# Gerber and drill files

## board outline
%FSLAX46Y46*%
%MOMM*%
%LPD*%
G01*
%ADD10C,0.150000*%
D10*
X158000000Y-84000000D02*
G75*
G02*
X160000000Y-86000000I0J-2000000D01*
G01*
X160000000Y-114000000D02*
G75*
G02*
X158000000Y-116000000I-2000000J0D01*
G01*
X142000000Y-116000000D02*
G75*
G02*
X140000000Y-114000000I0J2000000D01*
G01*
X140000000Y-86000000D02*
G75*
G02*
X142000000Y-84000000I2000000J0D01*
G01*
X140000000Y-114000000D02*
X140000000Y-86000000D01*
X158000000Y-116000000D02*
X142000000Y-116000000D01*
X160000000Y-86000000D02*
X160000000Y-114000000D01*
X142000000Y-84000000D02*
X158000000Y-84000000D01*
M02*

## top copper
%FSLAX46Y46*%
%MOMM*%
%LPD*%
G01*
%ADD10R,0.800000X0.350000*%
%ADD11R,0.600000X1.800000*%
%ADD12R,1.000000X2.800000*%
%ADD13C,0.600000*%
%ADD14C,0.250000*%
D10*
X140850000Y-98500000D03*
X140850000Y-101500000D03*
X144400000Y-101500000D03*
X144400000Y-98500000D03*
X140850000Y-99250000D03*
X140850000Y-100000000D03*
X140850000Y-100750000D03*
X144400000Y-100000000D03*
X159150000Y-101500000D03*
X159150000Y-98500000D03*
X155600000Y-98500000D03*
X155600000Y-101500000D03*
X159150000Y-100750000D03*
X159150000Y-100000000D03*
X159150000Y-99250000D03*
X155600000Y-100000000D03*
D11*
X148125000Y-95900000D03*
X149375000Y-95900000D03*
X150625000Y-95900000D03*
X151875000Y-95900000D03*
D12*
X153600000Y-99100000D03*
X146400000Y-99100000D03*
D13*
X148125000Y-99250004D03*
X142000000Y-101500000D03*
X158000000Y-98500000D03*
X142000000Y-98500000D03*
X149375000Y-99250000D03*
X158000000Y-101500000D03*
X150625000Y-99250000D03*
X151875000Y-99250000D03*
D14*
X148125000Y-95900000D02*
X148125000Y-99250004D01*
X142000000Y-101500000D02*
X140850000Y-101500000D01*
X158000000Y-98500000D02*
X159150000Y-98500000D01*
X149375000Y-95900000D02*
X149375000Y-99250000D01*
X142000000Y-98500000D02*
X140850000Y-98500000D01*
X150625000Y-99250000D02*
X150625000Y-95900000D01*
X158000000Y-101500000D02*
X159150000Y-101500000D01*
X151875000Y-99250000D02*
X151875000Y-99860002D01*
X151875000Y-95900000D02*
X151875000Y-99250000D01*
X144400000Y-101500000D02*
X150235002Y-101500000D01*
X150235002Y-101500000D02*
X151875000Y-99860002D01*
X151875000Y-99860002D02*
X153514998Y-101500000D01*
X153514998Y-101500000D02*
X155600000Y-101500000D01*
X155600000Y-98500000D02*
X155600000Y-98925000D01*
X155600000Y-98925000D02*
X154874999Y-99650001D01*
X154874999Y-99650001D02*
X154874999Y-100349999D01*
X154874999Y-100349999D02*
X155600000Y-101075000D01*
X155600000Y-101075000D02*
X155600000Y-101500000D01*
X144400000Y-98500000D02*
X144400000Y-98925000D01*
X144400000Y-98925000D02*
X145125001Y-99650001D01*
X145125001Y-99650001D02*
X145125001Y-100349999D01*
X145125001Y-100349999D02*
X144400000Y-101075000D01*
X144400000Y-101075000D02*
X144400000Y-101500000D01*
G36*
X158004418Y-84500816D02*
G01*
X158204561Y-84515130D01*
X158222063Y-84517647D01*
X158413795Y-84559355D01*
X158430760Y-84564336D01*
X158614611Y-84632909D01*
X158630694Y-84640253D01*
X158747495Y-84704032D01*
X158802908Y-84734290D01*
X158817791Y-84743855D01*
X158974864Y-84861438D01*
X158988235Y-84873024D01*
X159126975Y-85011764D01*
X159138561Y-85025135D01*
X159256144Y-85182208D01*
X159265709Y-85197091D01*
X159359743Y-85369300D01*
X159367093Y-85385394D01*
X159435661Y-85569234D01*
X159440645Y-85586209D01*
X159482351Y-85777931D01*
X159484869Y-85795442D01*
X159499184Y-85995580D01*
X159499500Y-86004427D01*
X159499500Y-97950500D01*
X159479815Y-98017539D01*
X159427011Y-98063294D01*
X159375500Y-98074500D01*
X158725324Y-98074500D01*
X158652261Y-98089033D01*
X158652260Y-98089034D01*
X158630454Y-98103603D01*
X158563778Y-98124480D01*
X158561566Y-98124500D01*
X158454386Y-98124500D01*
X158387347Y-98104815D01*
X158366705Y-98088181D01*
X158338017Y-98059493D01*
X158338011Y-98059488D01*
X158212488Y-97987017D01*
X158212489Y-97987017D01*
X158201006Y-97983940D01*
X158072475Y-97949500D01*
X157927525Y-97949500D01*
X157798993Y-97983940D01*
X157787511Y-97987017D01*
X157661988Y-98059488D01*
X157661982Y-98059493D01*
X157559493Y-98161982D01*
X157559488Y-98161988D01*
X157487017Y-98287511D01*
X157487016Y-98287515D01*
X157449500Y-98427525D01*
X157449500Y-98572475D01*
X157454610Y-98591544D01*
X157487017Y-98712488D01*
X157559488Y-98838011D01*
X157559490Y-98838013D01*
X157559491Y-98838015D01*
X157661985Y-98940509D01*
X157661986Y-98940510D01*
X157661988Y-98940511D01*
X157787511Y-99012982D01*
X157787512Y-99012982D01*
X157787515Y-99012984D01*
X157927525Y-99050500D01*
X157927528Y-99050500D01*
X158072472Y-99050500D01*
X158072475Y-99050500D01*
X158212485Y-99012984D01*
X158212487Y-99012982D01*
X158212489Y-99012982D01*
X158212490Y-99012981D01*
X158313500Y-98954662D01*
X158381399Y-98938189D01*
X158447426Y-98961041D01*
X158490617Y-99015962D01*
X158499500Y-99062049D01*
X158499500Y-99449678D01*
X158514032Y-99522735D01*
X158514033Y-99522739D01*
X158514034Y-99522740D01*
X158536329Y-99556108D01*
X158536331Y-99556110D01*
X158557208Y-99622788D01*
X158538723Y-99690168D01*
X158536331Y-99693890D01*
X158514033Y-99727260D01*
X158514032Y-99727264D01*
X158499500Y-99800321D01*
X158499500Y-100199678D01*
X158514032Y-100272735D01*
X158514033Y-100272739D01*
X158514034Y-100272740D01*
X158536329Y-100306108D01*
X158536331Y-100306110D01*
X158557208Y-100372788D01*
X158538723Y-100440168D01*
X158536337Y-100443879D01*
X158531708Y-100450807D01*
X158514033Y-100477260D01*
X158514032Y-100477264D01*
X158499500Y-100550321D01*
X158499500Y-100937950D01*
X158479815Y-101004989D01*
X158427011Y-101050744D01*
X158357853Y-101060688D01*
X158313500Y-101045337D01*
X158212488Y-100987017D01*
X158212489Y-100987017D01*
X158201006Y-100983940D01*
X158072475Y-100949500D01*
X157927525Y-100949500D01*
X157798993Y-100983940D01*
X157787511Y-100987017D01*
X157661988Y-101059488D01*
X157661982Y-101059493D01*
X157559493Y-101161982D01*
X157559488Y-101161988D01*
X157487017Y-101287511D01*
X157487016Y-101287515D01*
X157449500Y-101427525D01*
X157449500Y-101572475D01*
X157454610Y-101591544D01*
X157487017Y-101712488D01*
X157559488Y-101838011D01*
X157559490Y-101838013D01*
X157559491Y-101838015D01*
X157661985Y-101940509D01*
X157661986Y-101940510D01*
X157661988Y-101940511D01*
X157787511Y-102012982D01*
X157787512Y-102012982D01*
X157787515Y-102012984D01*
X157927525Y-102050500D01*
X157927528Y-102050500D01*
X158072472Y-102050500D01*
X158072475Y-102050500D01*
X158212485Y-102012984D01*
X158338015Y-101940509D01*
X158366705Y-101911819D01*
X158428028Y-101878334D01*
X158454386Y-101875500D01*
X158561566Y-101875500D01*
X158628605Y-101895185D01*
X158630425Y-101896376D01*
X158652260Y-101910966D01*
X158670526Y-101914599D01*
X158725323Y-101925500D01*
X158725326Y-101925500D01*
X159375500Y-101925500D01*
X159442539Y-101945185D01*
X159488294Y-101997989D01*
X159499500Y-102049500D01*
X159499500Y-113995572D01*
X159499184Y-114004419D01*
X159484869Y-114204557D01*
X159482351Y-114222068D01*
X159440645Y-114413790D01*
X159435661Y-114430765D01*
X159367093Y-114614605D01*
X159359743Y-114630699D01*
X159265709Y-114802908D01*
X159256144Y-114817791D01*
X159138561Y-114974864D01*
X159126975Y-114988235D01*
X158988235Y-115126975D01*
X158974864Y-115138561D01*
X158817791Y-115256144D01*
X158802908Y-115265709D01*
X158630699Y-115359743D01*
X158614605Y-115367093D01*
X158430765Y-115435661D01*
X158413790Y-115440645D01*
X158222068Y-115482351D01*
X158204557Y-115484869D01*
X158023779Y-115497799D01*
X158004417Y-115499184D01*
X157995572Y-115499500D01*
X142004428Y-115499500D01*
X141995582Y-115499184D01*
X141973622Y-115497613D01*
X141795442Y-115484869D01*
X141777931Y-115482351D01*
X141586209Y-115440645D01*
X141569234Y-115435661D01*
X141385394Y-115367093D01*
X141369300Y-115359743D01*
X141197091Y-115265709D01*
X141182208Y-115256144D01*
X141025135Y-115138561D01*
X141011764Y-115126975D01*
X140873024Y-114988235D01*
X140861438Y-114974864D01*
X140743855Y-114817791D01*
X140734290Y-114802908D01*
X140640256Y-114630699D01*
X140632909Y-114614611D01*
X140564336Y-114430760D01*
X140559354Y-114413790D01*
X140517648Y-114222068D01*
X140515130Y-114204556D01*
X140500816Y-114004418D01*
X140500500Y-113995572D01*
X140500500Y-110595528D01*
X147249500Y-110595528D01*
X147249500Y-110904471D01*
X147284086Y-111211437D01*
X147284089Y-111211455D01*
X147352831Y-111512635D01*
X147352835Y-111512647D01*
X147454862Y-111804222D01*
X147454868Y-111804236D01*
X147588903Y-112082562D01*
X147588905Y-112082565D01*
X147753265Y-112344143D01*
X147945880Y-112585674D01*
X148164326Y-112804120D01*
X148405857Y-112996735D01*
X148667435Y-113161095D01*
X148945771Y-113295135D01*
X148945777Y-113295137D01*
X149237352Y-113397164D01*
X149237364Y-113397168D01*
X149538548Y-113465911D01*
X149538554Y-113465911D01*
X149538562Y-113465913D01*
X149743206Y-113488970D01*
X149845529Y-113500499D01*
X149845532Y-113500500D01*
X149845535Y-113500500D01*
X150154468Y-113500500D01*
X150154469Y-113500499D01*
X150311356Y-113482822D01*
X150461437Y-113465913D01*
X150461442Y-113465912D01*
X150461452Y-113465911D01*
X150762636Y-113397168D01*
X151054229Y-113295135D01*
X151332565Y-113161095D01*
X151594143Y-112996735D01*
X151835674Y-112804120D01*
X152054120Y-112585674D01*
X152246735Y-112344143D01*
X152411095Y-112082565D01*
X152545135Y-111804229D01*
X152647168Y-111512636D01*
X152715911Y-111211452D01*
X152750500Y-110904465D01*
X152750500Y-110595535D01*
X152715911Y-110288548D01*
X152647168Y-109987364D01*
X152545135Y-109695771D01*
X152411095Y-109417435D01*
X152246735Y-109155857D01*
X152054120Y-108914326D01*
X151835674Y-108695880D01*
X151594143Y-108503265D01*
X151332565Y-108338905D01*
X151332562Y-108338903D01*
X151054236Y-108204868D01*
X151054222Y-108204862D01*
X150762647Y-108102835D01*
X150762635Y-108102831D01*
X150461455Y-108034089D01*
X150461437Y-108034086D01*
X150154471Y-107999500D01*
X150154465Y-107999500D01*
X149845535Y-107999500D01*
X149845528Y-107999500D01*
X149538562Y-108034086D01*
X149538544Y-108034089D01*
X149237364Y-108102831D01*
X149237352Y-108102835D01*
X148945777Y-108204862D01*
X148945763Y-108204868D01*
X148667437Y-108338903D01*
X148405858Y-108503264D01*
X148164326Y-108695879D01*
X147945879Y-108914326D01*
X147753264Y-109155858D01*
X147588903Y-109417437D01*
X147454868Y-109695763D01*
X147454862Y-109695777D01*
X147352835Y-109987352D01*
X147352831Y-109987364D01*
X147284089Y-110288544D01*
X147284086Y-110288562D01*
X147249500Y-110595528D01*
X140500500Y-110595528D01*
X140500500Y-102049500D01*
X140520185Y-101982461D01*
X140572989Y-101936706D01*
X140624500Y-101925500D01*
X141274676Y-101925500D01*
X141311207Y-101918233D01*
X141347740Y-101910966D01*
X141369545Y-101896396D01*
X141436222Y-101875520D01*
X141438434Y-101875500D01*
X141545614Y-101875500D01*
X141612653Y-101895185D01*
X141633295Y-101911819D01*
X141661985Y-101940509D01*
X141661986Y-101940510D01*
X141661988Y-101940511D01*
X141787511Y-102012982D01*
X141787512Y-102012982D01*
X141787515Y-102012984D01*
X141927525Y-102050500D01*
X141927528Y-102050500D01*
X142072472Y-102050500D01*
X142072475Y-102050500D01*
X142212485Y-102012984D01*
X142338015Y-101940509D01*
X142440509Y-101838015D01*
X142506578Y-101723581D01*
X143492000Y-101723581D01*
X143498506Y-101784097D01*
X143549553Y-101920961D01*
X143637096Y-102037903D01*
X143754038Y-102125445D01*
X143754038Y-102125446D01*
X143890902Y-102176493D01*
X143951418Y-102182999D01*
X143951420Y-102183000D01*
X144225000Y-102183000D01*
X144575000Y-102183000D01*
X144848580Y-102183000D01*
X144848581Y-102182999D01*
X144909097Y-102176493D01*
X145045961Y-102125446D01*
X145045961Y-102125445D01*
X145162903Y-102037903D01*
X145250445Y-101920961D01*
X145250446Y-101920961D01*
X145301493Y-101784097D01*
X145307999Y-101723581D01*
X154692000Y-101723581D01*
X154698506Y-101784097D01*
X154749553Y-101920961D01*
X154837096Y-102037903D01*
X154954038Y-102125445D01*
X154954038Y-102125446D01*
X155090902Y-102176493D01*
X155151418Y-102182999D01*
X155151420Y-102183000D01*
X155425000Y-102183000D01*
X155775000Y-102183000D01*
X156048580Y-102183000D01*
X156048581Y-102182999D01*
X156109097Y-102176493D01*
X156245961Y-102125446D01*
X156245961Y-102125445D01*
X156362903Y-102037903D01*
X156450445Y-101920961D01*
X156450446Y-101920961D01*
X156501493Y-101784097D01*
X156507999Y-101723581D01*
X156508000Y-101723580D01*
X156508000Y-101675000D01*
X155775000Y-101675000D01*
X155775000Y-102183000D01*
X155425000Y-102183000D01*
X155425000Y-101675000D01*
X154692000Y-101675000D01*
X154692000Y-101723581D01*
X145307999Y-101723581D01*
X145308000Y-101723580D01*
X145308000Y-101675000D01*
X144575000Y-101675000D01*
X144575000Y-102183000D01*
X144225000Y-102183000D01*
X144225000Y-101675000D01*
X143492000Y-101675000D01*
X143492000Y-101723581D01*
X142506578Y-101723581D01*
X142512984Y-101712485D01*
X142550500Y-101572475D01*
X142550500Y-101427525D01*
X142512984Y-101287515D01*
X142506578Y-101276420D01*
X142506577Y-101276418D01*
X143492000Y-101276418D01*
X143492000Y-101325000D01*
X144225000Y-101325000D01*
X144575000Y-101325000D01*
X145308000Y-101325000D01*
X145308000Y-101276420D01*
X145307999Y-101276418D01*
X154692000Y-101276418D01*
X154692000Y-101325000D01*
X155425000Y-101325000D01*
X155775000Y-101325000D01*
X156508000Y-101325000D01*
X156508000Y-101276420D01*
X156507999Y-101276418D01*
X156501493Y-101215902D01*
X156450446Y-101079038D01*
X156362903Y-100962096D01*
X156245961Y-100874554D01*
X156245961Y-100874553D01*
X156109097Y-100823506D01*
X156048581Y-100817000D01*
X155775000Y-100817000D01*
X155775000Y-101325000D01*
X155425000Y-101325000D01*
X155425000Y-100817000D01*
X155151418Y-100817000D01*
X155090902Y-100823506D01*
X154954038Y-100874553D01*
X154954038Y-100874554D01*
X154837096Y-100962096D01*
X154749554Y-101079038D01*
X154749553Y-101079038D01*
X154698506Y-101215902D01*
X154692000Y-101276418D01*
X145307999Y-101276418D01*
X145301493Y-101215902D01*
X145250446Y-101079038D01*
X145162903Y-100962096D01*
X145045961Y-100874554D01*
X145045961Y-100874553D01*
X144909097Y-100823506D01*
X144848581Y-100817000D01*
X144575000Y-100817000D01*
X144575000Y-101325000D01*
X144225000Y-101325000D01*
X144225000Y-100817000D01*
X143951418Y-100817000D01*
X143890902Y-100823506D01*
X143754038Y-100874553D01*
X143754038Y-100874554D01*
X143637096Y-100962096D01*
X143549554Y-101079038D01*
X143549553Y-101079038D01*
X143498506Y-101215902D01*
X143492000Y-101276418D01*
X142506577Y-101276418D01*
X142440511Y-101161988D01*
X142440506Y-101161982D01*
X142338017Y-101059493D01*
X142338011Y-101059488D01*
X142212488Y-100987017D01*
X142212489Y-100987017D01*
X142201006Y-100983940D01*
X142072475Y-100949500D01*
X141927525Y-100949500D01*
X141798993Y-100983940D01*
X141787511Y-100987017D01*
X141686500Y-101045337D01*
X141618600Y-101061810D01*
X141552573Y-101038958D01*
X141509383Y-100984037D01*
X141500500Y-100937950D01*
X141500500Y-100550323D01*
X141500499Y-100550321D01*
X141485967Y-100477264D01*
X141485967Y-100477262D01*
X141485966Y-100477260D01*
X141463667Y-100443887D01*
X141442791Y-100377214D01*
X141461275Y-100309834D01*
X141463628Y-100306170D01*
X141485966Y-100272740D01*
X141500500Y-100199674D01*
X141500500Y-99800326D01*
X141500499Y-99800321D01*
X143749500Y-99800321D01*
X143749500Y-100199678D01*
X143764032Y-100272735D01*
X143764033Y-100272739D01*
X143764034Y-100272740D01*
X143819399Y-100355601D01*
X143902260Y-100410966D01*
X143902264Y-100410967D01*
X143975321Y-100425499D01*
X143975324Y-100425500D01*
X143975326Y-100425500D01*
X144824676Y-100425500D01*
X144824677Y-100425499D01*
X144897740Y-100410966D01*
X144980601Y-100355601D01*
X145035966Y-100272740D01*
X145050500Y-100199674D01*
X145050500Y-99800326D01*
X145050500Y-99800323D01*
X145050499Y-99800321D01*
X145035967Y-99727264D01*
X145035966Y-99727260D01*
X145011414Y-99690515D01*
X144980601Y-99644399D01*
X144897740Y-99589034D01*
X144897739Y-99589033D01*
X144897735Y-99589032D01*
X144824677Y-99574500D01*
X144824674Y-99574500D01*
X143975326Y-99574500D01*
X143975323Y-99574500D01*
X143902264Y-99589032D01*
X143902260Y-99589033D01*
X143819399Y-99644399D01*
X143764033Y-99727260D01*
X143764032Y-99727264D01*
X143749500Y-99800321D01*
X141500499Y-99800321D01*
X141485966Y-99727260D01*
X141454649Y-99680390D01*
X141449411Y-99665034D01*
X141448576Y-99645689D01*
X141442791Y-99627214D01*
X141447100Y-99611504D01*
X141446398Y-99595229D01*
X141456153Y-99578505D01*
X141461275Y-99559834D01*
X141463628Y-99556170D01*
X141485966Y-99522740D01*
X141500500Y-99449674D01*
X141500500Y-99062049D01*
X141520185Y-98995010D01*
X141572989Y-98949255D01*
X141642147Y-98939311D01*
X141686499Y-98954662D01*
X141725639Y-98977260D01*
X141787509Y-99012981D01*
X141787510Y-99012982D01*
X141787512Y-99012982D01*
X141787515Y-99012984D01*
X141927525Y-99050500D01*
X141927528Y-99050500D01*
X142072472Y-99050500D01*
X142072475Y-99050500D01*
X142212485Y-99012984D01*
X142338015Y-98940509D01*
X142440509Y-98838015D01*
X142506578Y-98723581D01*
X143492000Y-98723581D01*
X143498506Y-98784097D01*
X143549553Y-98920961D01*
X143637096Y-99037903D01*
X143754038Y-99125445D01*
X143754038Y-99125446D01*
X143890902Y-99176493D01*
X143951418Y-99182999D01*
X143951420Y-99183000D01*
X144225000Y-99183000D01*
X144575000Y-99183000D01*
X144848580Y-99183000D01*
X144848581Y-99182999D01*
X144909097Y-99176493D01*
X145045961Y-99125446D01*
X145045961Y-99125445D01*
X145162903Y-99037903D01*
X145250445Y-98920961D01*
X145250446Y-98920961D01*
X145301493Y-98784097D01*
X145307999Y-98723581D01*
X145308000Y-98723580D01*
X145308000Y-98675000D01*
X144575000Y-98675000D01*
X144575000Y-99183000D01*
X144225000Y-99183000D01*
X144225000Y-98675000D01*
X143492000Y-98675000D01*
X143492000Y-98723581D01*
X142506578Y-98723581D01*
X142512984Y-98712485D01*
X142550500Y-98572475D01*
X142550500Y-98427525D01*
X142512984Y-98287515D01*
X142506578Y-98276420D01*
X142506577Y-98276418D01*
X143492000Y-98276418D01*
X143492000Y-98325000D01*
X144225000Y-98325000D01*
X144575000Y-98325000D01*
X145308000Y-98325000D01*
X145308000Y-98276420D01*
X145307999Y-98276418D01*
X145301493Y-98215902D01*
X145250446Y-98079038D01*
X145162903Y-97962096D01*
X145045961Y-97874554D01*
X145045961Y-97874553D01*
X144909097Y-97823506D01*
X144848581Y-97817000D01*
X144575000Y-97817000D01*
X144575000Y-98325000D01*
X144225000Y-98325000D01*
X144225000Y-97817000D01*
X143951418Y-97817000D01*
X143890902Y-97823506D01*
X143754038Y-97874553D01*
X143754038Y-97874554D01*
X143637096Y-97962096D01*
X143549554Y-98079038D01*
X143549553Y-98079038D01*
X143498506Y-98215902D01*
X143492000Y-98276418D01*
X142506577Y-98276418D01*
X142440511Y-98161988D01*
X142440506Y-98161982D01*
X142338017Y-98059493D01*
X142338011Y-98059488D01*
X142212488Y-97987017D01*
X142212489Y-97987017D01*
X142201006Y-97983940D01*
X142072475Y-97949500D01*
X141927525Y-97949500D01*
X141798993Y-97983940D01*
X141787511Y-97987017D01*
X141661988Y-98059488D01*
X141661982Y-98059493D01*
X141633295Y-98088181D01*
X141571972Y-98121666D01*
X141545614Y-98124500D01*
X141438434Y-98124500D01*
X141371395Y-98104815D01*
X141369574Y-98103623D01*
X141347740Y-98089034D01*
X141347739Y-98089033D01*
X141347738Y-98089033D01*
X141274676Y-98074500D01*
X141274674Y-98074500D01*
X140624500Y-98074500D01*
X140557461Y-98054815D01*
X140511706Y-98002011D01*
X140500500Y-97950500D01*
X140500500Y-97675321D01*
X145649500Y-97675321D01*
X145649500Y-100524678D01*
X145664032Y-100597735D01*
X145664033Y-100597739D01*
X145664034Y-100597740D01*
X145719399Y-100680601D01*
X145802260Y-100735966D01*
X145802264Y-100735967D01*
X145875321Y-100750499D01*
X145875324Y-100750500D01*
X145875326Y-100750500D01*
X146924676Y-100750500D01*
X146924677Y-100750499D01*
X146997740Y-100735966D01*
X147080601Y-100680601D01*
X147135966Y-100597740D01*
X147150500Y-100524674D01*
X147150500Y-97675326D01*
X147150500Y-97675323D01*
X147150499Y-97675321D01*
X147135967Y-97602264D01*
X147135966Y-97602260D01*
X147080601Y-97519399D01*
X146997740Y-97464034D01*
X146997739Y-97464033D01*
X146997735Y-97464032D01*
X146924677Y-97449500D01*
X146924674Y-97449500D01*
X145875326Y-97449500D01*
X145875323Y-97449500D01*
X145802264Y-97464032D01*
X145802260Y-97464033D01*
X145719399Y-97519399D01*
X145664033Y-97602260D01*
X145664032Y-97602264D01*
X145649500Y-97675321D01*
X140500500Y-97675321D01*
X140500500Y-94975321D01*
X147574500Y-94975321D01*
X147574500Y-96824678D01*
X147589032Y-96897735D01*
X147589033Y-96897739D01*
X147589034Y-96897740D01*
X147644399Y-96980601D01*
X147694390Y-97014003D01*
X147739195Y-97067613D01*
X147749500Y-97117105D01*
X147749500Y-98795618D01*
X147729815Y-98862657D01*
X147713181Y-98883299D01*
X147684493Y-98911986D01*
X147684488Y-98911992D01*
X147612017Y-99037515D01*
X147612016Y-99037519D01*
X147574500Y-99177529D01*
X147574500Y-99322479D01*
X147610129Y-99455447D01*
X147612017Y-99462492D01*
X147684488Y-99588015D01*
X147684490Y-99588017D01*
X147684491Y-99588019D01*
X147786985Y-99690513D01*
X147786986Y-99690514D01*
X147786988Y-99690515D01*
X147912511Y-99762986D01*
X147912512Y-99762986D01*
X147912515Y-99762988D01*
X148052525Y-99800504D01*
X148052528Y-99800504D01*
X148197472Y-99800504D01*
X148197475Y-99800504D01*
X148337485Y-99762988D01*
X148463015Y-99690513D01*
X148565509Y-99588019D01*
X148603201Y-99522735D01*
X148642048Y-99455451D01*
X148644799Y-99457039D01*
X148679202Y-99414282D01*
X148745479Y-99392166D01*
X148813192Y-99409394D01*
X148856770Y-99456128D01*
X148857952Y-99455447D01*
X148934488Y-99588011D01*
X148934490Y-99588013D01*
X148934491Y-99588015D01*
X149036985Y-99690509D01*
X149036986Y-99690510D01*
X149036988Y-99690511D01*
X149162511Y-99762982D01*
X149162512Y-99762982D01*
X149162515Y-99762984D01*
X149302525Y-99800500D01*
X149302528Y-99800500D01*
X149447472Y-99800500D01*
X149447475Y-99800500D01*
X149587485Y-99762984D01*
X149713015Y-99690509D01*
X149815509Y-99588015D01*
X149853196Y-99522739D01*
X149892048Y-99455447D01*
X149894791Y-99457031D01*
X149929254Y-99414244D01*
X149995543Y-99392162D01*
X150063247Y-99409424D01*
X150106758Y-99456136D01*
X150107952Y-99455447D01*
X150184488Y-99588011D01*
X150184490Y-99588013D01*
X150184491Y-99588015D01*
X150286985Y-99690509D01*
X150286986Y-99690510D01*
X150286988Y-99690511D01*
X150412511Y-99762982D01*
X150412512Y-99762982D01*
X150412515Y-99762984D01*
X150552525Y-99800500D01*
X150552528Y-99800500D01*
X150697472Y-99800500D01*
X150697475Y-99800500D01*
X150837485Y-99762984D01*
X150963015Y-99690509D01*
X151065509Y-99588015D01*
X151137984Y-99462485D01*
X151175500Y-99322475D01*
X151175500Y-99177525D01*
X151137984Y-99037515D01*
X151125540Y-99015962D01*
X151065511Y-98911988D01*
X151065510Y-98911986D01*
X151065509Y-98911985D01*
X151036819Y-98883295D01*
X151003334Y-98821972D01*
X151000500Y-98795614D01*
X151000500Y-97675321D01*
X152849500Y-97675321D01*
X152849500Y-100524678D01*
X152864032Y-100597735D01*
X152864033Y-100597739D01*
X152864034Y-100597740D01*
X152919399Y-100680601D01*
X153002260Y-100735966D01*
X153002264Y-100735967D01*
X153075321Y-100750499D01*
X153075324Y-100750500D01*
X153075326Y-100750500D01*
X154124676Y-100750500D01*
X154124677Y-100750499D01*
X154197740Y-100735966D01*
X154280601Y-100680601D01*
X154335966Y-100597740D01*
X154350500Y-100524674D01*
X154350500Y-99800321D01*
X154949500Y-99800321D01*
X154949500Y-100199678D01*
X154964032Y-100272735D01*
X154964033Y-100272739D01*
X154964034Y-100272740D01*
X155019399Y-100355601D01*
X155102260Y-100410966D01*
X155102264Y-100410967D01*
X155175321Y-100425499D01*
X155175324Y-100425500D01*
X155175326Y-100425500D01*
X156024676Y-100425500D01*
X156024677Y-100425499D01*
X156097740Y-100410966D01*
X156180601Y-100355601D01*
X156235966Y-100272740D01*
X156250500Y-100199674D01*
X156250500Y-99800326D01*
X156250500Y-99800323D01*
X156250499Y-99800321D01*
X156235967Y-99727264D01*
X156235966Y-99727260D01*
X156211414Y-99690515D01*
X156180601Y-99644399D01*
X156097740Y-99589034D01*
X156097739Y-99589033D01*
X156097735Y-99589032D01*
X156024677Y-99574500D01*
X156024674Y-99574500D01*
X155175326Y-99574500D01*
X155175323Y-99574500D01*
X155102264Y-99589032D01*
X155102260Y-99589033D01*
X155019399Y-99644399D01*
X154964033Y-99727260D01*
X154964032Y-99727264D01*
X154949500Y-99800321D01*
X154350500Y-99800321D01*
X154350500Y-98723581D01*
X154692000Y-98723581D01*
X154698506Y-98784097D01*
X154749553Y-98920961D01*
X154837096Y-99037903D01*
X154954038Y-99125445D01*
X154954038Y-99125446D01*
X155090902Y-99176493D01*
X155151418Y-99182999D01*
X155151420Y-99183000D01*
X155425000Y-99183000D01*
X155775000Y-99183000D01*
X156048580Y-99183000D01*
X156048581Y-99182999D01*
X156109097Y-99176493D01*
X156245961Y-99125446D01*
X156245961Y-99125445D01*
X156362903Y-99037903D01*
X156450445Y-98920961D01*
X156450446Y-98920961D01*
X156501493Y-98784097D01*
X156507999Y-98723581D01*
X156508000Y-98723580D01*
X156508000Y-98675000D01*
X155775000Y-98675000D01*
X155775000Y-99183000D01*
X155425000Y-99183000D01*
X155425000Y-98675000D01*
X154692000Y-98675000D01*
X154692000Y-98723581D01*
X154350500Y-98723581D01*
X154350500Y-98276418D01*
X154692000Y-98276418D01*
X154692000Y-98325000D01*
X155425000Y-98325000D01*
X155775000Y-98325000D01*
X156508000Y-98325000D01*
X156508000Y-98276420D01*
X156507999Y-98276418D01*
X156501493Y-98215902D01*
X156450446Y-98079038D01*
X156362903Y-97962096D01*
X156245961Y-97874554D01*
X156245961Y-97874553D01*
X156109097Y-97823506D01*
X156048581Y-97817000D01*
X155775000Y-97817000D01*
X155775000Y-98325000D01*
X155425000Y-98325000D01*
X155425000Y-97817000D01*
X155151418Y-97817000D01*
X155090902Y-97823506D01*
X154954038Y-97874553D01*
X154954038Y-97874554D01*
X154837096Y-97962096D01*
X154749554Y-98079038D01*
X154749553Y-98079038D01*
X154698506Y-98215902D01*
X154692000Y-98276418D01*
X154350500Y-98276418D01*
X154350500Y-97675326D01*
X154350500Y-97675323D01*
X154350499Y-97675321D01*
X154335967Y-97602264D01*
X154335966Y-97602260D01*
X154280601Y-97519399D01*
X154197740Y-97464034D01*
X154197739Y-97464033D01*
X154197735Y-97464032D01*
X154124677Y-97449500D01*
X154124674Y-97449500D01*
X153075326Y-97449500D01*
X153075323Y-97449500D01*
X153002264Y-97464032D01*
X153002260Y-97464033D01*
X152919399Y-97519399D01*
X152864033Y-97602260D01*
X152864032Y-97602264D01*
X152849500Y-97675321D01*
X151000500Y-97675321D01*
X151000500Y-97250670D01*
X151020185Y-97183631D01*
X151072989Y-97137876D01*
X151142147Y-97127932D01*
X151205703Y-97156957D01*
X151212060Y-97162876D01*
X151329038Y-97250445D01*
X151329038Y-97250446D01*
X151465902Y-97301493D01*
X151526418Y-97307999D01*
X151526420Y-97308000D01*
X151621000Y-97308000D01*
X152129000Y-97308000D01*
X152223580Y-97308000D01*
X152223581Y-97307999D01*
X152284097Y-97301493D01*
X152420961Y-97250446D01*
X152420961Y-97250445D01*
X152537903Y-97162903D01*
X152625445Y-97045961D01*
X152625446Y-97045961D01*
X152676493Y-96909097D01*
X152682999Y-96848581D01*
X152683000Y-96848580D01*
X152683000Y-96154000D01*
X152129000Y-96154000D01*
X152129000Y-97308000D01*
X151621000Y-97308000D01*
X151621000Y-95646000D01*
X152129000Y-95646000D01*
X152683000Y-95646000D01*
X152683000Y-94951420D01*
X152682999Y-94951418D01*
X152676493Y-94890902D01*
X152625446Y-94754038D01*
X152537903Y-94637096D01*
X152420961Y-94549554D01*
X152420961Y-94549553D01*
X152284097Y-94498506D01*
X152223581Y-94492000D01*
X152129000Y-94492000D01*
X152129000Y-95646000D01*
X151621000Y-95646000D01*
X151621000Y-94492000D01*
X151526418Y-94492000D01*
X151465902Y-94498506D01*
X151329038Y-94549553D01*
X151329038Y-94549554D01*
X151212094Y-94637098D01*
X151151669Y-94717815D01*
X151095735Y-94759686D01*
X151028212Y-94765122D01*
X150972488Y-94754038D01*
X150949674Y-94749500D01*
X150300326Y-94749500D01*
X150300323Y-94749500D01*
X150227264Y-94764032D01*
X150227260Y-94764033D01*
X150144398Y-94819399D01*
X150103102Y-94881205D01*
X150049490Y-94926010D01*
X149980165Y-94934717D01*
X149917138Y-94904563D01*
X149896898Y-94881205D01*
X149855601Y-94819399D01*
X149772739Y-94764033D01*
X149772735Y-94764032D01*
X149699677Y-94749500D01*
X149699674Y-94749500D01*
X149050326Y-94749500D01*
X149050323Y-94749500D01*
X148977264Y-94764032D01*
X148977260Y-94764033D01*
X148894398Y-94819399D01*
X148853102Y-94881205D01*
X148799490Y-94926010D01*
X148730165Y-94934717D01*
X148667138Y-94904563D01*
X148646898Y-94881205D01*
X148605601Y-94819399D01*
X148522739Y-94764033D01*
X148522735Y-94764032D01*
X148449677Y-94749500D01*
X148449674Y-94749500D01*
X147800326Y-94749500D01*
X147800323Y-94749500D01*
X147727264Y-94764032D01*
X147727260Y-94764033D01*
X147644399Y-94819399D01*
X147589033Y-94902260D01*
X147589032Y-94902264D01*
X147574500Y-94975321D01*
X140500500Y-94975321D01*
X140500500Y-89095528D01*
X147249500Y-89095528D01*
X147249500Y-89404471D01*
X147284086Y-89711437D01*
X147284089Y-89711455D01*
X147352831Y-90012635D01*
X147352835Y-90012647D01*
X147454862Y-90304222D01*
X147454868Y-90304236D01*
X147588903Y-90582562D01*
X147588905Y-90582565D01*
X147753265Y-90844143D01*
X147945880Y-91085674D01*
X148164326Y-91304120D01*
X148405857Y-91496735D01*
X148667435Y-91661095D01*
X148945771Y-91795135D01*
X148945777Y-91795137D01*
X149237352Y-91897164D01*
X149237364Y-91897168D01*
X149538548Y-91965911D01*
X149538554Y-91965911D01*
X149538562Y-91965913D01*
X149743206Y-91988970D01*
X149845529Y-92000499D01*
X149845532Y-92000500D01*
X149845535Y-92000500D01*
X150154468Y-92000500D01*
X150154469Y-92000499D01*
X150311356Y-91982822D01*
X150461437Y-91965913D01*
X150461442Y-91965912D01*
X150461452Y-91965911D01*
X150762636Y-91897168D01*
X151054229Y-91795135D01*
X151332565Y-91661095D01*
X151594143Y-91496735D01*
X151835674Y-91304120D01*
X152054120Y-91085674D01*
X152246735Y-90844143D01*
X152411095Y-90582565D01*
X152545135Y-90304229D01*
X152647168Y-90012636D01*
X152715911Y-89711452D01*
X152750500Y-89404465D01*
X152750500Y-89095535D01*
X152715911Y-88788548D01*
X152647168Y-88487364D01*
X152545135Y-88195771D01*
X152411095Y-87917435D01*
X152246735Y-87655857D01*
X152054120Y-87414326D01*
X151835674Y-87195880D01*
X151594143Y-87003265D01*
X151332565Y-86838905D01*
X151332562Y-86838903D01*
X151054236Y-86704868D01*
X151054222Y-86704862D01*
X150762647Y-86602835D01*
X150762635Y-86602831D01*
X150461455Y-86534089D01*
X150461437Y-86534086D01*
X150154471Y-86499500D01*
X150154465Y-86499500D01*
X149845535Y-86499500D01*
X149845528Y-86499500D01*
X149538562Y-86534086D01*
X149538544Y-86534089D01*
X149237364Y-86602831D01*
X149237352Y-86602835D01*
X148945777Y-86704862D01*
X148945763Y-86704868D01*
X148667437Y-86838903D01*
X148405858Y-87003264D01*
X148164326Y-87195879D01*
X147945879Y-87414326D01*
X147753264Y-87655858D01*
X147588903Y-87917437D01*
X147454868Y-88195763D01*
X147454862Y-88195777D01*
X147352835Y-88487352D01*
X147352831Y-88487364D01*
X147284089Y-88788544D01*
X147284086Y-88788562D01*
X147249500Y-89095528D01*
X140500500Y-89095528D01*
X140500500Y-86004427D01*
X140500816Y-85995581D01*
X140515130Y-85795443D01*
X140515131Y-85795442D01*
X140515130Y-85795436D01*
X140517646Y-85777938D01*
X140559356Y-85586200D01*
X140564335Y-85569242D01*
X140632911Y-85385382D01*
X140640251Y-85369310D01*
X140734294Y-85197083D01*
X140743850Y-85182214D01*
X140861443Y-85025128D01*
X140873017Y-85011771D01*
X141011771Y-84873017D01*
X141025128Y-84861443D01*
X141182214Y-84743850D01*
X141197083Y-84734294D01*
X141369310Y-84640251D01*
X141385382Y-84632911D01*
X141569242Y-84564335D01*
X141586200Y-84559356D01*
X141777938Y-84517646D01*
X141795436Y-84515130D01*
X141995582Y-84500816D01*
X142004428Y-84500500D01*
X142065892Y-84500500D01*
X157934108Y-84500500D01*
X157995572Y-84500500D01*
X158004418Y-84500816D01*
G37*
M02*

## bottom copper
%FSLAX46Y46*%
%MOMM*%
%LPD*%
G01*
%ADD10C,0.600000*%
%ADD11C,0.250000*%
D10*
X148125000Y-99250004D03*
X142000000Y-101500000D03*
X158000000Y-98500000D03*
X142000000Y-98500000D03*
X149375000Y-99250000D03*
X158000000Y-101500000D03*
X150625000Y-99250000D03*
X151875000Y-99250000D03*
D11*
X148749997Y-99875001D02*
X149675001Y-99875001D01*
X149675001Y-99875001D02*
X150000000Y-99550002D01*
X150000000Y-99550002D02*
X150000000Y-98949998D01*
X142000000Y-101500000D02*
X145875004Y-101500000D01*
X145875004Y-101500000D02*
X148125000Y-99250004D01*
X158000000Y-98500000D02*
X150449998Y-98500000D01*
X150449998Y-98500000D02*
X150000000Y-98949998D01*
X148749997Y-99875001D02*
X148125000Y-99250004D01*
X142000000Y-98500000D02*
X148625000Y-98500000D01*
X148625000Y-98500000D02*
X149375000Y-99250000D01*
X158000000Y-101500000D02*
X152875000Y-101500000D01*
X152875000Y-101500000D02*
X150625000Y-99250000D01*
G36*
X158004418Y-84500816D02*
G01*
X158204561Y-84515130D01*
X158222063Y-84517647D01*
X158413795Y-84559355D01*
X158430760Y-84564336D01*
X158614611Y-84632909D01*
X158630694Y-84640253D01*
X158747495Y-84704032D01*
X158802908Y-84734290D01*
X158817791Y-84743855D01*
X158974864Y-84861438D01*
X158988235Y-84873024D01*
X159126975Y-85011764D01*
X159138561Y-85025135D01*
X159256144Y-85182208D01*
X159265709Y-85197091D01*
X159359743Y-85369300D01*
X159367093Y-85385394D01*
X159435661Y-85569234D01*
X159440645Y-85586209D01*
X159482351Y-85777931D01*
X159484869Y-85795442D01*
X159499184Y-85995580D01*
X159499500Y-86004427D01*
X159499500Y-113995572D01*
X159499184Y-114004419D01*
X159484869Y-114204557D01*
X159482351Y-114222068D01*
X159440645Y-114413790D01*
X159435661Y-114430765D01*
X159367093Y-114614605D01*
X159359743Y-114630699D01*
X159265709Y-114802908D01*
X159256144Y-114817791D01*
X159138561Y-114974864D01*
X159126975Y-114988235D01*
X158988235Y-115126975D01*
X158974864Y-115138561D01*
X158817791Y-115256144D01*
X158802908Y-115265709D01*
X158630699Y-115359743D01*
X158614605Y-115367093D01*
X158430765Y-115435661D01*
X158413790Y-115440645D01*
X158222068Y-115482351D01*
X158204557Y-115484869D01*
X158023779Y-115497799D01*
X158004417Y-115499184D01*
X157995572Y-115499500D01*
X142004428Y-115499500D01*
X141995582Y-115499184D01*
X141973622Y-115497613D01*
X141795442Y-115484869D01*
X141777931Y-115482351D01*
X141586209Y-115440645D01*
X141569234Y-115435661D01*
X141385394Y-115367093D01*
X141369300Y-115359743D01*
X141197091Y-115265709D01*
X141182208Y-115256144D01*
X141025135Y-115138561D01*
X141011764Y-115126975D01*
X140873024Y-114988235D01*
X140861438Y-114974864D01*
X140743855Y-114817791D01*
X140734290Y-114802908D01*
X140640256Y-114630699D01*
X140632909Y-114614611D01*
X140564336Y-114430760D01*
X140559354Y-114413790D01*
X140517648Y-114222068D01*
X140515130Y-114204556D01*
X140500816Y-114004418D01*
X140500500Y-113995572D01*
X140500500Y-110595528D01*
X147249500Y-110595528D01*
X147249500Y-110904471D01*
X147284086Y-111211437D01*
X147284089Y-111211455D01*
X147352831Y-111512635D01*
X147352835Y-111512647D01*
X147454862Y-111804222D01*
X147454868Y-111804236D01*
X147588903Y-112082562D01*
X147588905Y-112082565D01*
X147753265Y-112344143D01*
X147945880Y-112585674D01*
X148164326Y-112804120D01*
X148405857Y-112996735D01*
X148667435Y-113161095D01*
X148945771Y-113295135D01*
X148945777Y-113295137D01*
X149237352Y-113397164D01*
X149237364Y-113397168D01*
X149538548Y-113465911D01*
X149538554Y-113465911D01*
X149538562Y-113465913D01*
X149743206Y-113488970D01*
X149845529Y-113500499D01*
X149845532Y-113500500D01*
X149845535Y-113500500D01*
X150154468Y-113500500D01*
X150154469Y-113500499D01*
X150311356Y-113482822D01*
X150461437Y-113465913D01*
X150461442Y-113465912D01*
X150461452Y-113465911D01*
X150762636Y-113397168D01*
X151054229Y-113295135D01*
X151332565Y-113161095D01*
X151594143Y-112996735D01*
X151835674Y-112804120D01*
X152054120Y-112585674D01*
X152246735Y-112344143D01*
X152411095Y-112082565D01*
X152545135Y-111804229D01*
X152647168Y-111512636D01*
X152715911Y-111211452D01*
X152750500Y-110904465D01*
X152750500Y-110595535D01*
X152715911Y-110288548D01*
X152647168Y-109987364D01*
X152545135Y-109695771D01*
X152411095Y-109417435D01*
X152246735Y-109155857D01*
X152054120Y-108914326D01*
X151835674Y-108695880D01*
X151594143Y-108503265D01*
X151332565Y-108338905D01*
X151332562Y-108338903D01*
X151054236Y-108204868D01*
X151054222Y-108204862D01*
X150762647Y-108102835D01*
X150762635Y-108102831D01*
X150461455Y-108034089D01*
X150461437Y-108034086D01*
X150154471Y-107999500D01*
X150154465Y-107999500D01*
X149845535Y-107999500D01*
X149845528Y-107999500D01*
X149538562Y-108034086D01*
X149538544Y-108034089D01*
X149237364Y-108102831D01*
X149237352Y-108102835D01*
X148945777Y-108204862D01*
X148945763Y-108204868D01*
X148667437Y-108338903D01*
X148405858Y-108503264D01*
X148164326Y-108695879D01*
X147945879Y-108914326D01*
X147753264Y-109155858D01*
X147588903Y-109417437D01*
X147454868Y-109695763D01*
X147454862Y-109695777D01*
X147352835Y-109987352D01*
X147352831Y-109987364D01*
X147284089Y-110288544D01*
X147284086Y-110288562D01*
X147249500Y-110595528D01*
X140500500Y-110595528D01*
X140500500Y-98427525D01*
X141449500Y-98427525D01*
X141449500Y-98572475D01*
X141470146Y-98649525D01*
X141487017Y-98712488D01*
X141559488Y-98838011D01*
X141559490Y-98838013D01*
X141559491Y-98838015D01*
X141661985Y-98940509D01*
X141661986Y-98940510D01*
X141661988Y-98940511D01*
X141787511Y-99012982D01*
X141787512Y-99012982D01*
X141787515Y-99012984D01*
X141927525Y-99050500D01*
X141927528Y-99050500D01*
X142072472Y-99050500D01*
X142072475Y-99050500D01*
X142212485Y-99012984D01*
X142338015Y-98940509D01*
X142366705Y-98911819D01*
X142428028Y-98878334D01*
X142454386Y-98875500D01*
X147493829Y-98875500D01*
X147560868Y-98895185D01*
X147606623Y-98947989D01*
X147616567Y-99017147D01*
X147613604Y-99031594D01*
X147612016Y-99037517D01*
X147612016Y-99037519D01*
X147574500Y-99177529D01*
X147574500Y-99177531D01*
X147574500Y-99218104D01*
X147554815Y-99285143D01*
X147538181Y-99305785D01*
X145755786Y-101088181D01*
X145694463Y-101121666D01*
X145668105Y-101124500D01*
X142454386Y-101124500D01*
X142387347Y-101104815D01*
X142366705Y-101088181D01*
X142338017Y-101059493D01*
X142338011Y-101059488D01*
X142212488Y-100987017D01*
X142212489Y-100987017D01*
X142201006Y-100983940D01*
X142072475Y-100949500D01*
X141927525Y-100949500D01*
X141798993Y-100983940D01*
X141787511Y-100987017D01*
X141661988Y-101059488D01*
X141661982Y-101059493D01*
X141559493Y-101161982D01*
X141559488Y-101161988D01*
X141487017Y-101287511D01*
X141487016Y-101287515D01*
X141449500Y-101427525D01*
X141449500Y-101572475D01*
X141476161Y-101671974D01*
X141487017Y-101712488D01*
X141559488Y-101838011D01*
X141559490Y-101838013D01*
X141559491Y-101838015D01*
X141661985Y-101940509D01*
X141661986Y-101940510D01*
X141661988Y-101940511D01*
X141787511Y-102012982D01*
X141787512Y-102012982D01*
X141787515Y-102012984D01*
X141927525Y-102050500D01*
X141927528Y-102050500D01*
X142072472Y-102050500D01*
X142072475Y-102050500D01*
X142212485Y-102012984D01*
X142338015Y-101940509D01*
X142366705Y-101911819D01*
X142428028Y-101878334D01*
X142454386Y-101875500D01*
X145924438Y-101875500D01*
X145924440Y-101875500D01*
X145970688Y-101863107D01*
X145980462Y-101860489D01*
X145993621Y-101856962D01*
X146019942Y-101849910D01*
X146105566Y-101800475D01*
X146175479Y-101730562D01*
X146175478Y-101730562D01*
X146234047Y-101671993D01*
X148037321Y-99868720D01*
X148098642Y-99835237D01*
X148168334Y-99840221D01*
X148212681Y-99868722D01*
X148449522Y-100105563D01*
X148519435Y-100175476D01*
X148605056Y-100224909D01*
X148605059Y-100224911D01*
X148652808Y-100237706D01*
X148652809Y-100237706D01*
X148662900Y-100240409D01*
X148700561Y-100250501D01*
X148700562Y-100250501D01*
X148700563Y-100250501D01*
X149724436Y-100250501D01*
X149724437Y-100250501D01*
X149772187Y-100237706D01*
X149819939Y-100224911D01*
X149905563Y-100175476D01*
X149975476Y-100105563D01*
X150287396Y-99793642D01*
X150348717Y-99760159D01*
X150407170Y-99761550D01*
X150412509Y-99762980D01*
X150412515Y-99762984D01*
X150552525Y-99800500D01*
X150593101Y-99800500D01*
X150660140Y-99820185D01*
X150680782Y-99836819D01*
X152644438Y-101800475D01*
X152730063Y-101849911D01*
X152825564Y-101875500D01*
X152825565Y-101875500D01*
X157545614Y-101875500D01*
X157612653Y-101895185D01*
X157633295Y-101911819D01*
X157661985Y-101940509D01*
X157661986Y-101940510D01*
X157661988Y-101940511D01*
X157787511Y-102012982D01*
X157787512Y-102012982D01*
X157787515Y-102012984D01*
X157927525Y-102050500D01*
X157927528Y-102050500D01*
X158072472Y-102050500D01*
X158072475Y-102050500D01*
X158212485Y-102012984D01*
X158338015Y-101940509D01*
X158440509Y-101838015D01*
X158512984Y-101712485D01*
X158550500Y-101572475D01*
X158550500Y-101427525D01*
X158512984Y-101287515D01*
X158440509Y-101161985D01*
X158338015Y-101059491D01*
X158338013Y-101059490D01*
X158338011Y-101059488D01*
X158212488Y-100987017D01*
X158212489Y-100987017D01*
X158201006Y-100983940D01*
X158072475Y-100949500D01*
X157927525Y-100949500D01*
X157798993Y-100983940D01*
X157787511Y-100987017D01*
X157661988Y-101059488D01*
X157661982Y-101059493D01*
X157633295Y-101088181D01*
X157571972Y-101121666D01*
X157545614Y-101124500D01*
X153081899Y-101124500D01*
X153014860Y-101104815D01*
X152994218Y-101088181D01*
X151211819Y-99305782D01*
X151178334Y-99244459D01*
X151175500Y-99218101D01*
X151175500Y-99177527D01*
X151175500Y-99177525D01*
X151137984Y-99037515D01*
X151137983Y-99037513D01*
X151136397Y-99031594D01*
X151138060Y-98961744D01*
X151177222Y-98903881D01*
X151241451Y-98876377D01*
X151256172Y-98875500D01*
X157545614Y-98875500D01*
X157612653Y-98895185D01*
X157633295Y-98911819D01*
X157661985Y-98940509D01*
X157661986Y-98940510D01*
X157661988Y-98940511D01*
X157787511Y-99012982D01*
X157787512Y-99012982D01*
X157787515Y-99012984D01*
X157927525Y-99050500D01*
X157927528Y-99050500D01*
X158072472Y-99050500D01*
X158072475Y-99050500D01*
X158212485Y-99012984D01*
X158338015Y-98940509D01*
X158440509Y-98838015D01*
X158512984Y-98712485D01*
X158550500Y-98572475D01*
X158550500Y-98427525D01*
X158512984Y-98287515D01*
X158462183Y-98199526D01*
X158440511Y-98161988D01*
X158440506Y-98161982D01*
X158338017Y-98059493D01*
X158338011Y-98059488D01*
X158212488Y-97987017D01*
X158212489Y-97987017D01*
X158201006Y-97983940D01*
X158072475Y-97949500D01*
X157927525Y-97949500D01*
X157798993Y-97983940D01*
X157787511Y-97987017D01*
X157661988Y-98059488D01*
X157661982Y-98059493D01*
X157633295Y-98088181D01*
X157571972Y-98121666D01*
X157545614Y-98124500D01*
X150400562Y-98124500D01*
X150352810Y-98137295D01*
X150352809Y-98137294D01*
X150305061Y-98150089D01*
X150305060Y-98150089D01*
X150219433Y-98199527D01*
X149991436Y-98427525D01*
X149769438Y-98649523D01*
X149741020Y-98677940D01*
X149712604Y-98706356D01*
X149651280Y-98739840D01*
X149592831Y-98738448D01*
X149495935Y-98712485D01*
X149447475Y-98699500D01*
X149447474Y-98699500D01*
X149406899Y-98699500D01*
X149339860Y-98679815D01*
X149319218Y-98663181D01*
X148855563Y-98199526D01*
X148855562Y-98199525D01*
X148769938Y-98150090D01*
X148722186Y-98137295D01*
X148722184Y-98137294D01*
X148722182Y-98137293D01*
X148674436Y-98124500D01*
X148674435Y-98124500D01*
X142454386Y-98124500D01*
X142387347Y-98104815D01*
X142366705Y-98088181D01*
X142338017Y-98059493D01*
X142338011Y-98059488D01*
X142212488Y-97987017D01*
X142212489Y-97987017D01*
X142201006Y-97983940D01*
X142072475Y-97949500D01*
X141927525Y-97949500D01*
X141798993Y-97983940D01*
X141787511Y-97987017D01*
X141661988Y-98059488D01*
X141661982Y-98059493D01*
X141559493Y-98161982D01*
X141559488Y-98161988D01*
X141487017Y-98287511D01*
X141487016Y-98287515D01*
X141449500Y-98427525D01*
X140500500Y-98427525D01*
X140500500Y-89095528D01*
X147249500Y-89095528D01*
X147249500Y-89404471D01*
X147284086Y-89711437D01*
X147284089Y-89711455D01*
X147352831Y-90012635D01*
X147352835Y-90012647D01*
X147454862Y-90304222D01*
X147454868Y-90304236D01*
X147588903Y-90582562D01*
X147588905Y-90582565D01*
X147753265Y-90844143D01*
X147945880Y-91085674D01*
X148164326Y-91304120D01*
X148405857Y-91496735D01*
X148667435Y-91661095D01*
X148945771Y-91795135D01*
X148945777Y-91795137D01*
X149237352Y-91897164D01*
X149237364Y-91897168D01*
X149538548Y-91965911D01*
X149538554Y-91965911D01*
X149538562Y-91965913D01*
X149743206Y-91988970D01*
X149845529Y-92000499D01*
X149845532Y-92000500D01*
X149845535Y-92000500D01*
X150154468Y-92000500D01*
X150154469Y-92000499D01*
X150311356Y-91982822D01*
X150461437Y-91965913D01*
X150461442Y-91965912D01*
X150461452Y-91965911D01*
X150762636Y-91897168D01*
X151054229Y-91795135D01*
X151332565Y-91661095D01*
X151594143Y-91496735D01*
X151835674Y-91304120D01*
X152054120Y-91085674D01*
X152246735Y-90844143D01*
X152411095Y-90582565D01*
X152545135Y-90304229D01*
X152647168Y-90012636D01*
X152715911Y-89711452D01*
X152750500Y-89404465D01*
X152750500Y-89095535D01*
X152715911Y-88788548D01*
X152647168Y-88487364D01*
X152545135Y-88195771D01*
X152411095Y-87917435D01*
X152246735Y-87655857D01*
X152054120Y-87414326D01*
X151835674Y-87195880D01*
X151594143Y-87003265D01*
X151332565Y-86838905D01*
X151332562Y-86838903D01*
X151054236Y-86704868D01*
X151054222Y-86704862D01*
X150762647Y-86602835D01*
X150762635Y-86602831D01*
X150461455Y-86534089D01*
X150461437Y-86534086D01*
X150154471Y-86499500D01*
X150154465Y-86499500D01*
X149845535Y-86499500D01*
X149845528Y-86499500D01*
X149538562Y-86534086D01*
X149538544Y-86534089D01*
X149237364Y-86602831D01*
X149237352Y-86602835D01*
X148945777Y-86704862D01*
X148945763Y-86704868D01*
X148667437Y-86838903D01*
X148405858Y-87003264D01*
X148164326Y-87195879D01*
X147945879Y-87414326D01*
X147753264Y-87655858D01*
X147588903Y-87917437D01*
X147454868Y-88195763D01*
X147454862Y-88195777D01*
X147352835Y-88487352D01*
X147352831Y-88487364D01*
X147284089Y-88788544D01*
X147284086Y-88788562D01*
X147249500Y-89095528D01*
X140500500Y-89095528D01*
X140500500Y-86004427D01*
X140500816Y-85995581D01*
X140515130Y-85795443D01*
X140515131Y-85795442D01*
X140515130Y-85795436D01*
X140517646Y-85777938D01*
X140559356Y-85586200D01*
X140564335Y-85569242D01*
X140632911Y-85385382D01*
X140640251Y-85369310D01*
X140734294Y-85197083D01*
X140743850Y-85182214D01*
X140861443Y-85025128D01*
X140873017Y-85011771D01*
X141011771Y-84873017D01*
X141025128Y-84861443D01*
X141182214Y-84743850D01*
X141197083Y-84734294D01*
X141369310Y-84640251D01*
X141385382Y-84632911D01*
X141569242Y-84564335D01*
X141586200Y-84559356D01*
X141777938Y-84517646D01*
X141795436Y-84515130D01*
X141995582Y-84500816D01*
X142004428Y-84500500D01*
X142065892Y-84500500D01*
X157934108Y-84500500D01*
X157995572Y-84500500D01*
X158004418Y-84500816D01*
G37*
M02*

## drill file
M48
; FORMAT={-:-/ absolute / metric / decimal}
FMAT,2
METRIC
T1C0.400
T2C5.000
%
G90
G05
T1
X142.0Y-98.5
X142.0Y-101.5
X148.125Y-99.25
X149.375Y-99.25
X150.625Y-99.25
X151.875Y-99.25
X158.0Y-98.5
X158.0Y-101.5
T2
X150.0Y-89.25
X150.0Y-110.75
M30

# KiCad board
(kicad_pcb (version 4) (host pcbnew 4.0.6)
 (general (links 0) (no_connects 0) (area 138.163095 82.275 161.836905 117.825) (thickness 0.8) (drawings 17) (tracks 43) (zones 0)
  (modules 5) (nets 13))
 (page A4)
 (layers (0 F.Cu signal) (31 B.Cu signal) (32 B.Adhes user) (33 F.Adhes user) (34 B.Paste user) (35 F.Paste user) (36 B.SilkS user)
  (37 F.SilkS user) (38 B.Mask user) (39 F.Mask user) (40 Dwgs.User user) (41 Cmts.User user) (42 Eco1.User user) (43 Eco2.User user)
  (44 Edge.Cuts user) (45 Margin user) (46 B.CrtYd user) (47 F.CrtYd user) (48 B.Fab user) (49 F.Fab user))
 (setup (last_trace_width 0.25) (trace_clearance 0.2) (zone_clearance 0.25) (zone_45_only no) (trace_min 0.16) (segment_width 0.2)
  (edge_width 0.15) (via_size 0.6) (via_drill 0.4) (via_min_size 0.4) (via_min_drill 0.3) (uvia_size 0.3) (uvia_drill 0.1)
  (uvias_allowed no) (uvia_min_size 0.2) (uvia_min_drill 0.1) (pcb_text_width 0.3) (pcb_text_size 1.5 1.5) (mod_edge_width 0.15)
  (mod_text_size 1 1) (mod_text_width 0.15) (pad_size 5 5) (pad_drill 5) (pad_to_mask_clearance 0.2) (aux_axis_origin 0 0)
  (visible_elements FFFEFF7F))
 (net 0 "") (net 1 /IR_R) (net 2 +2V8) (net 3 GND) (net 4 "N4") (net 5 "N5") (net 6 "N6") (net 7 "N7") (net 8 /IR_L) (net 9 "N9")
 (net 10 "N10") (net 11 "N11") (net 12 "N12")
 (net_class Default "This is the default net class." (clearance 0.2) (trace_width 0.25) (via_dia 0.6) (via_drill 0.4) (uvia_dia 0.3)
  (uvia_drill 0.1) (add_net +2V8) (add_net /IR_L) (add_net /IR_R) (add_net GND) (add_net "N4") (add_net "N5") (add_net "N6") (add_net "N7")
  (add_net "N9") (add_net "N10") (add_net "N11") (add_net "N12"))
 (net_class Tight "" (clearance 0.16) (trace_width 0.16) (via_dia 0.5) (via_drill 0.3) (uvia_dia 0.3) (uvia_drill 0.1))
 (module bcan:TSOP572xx (layer F.Cu) (at 142.625 100)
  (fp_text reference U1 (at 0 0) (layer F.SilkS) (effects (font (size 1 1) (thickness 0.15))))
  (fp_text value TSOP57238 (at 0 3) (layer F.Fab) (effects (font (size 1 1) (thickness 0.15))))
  (pad 1 smd rect (at -1.775 -1.5) (size 0.8 0.35) (layers F.Cu F.Paste F.Mask) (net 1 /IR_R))
  (pad 5 smd rect (at -1.775 1.5) (size 0.8 0.35) (layers F.Cu F.Paste F.Mask) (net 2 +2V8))
  (pad 6 smd rect (at 1.775 1.5) (size 0.8 0.35) (layers F.Cu F.Paste F.Mask) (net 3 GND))
  (pad 8 smd rect (at 1.775 -1.5) (size 0.8 0.35) (layers F.Cu F.Paste F.Mask) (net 3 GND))
  (pad 2 smd rect (at -1.775 -0.75) (size 0.8 0.35) (layers F.Cu F.Mask) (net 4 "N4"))
  (pad 3 smd rect (at -1.775 0) (size 0.8 0.35) (layers F.Cu F.Mask) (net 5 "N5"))
  (pad 4 smd rect (at -1.775 0.75) (size 0.8 0.35) (layers F.Cu F.Mask) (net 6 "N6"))
  (pad 7 smd rect (at 1.775 0) (size 0.8 0.35) (layers F.Cu F.Mask) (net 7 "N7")))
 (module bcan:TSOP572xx (layer F.Cu) (at 157.375 100 180)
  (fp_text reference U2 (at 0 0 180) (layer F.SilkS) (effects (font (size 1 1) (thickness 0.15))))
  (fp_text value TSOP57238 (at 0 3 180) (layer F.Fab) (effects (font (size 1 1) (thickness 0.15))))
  (pad 1 smd rect (at -1.775 -1.5 180) (size 0.8 0.35) (layers F.Cu F.Paste F.Mask) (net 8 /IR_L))
  (pad 5 smd rect (at -1.775 1.5 180) (size 0.8 0.35) (layers F.Cu F.Paste F.Mask) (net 2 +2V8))
  (pad 6 smd rect (at 1.775 1.5 180) (size 0.8 0.35) (layers F.Cu F.Paste F.Mask) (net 3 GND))
  (pad 8 smd rect (at 1.775 -1.5 180) (size 0.8 0.35) (layers F.Cu F.Paste F.Mask) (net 3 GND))
  (pad 2 smd rect (at -1.775 -0.75 180) (size 0.8 0.35) (layers F.Cu F.Mask) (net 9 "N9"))
  (pad 3 smd rect (at -1.775 0 180) (size 0.8 0.35) (layers F.Cu F.Mask) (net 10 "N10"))
  (pad 4 smd rect (at -1.775 0.75 180) (size 0.8 0.35) (layers F.Cu F.Mask) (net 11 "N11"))
  (pad 7 smd rect (at 1.775 0 180) (size 0.8 0.35) (layers F.Cu F.Mask) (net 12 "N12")))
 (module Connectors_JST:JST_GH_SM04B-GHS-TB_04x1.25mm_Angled (layer F.Cu) (at 150 97.5)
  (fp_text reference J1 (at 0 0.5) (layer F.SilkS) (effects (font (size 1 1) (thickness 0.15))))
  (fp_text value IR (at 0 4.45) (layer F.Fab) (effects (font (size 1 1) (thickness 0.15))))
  (pad 1 smd rect (at -1.875 -1.6) (size 0.6 1.8) (layers F.Cu F.Paste F.Mask) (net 2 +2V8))
  (pad 2 smd rect (at -0.625 -1.6) (size 0.6 1.8) (layers F.Cu F.Paste F.Mask) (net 1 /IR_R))
  (pad 3 smd rect (at 0.625 -1.6) (size 0.6 1.8) (layers F.Cu F.Paste F.Mask) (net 8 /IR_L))
  (pad 4 smd rect (at 1.875 -1.6) (size 0.6 1.8) (layers F.Cu F.Paste F.Mask) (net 3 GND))
  (pad "" smd rect (at 3.6 1.6) (size 1 2.8) (layers F.Cu F.Paste F.Mask))
  (pad "" smd rect (at -3.6 1.6) (size 1 2.8) (layers F.Cu F.Paste F.Mask)))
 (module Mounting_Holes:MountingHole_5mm (layer F.Cu) (at 150 89.25)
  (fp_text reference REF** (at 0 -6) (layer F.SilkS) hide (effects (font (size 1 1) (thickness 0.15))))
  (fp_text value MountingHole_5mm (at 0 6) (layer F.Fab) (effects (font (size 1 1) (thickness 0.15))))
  (pad 1 np_thru_hole circle (at 0 0) (size 5 5) (drill 5) (layers *.Cu *.Mask)))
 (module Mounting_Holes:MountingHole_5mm (layer F.Cu) (at 150 110.75)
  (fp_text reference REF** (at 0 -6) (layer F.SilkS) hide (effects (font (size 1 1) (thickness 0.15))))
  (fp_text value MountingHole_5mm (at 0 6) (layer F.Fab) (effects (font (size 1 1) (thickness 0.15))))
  (pad 1 np_thru_hole circle (at 0 0) (size 5 5) (drill 5) (layers *.Cu *.Mask)))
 (gr_arc (start 158 86) (end 158 84) (angle 90) (layer Edge.Cuts) (width 0.15))
 (gr_arc (start 158 114) (end 160 114) (angle 90) (layer Edge.Cuts) (width 0.15))
 (gr_arc (start 142 114) (end 142 116) (angle 90) (layer Edge.Cuts) (width 0.15))
 (gr_arc (start 142 86) (end 140 86) (angle 90) (layer Edge.Cuts) (width 0.15))
 (gr_line (start 140 114) (end 140 86) (layer Edge.Cuts) (width 0.15))
 (gr_line (start 158 116) (end 142 116) (layer Edge.Cuts) (width 0.15))
 (gr_line (start 160 86) (end 160 114) (layer Edge.Cuts) (width 0.15))
 (gr_line (start 142 84) (end 158 84) (layer Edge.Cuts) (width 0.15))
 (segment (start 148.749997 99.875001) (end 149.675001 99.875001) (width 0.25) (layer B.Cu) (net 2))
 (segment (start 149.675001 99.875001) (end 150 99.550002) (width 0.25) (layer B.Cu) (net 2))
 (segment (start 150 99.550002) (end 150 98.949998) (width 0.25) (layer B.Cu) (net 2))
 (segment (start 142 101.5) (end 145.875004 101.5) (width 0.25) (layer B.Cu) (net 2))
 (segment (start 145.875004 101.5) (end 148.125 99.250004) (width 0.25) (layer B.Cu) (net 2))
 (segment (start 158 98.5) (end 150.449998 98.5) (width 0.25) (layer B.Cu) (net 2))
 (segment (start 150.449998 98.5) (end 150 98.949998) (width 0.25) (layer B.Cu) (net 2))
 (segment (start 148.749997 99.875001) (end 148.125 99.250004) (width 0.25) (layer B.Cu) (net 2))
 (segment (start 148.125 95.9) (end 148.125 99.250004) (width 0.25) (layer F.Cu) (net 2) (status 10))
 (via (at 148.125 99.250004) (size 0.6) (drill 0.4) (layers F.Cu B.Cu) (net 2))
 (segment (start 142 101.5) (end 140.85 101.5) (width 0.25) (layer F.Cu) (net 2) (status 20))
 (via (at 142 101.5) (size 0.6) (drill 0.4) (layers F.Cu B.Cu) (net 2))
 (segment (start 158 98.5) (end 159.15 98.5) (width 0.25) (layer F.Cu) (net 2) (status 20))
 (via (at 158 98.5) (size 0.6) (drill 0.4) (layers F.Cu B.Cu) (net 2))
 (segment (start 142 98.5) (end 148.625 98.5) (width 0.25) (layer B.Cu) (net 1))
 (segment (start 148.625 98.5) (end 149.375 99.25) (width 0.25) (layer B.Cu) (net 1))
 (segment (start 149.375 95.9) (end 149.375 99.25) (width 0.25) (layer F.Cu) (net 1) (status 10))
 (segment (start 142 98.5) (end 140.85 98.5) (width 0.25) (layer F.Cu) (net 1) (status 20))
 (via (at 142 98.5) (size 0.6) (drill 0.4) (layers F.Cu B.Cu) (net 1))
 (via (at 149.375 99.25) (size 0.6) (drill 0.4) (layers F.Cu B.Cu) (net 1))
 (segment (start 150.625 99.25) (end 150.625 95.9) (width 0.25) (layer F.Cu) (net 8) (status 20))
 (segment (start 158 101.5) (end 152.875 101.5) (width 0.25) (layer B.Cu) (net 8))
 (segment (start 152.875 101.5) (end 150.625 99.25) (width 0.25) (layer B.Cu) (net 8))
 (segment (start 158 101.5) (end 159.15 101.5) (width 0.25) (layer F.Cu) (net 8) (status 20))
 (via (at 158 101.5) (size 0.6) (drill 0.4) (layers F.Cu B.Cu) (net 8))
 (via (at 150.625 99.25) (size 0.6) (drill 0.4) (layers F.Cu B.Cu) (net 8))
 (segment (start 151.875 99.25) (end 151.875 99.860002) (width 0.25) (layer F.Cu) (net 3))
 (segment (start 151.875 95.9) (end 151.875 99.25) (width 0.25) (layer F.Cu) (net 3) (status 10))
 (via (at 151.875 99.25) (size 0.6) (drill 0.4) (layers F.Cu B.Cu) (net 3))
 (segment (start 144.4 101.5) (end 150.235002 101.5) (width 0.25) (layer F.Cu) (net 3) (status 10))
 (segment (start 150.235002 101.5) (end 151.875 99.860002) (width 0.25) (layer F.Cu) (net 3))
 (segment (start 151.875 99.860002) (end 153.514998 101.5) (width 0.25) (layer F.Cu) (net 3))
 (segment (start 153.514998 101.5) (end 155.6 101.5) (width 0.25) (layer F.Cu) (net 3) (status 20))
 (segment (start 155.6 98.5) (end 155.6 98.925) (width 0.25) (layer F.Cu) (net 3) (status 10))
 (segment (start 155.6 98.925) (end 154.874999 99.650001) (width 0.25) (layer F.Cu) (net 3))
 (segment (start 154.874999 99.650001) (end 154.874999 100.349999) (width 0.25) (layer F.Cu) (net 3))
 (segment (start 154.874999 100.349999) (end 155.6 101.075) (width 0.25) (layer F.Cu) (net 3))
 (segment (start 155.6 101.075) (end 155.6 101.5) (width 0.25) (layer F.Cu) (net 3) (status 20))
 (segment (start 144.4 98.5) (end 144.4 98.925) (width 0.25) (layer F.Cu) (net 3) (status 10))
 (segment (start 144.4 98.925) (end 145.125001 99.650001) (width 0.25) (layer F.Cu) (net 3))
 (segment (start 145.125001 99.650001) (end 145.125001 100.349999) (width 0.25) (layer F.Cu) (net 3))
 (segment (start 145.125001 100.349999) (end 144.4 101.075) (width 0.25) (layer F.Cu) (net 3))
 (segment (start 144.4 101.075) (end 144.4 101.5) (width 0.25) (layer F.Cu) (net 3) (status 20))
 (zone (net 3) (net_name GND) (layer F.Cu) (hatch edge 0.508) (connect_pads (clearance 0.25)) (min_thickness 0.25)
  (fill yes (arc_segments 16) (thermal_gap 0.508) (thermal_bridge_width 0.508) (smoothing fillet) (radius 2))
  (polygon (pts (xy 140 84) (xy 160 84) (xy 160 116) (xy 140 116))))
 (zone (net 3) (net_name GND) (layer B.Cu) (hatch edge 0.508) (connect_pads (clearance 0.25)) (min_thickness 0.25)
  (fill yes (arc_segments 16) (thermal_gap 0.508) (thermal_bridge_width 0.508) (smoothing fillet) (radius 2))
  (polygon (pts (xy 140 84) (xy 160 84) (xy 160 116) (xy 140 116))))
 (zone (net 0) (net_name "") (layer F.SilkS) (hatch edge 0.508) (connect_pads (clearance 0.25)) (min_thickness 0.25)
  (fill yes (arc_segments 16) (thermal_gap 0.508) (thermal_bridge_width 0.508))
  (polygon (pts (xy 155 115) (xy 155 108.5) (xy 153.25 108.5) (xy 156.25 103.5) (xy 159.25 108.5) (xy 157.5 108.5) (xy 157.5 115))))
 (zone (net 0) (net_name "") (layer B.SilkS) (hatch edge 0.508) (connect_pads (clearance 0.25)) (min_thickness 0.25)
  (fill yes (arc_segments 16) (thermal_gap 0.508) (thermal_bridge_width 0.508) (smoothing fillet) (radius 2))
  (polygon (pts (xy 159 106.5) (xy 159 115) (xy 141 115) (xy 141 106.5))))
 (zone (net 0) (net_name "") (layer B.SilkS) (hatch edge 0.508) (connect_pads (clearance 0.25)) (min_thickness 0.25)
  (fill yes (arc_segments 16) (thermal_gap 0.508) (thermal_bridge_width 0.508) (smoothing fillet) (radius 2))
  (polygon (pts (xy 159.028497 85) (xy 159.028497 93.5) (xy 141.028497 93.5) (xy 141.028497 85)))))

